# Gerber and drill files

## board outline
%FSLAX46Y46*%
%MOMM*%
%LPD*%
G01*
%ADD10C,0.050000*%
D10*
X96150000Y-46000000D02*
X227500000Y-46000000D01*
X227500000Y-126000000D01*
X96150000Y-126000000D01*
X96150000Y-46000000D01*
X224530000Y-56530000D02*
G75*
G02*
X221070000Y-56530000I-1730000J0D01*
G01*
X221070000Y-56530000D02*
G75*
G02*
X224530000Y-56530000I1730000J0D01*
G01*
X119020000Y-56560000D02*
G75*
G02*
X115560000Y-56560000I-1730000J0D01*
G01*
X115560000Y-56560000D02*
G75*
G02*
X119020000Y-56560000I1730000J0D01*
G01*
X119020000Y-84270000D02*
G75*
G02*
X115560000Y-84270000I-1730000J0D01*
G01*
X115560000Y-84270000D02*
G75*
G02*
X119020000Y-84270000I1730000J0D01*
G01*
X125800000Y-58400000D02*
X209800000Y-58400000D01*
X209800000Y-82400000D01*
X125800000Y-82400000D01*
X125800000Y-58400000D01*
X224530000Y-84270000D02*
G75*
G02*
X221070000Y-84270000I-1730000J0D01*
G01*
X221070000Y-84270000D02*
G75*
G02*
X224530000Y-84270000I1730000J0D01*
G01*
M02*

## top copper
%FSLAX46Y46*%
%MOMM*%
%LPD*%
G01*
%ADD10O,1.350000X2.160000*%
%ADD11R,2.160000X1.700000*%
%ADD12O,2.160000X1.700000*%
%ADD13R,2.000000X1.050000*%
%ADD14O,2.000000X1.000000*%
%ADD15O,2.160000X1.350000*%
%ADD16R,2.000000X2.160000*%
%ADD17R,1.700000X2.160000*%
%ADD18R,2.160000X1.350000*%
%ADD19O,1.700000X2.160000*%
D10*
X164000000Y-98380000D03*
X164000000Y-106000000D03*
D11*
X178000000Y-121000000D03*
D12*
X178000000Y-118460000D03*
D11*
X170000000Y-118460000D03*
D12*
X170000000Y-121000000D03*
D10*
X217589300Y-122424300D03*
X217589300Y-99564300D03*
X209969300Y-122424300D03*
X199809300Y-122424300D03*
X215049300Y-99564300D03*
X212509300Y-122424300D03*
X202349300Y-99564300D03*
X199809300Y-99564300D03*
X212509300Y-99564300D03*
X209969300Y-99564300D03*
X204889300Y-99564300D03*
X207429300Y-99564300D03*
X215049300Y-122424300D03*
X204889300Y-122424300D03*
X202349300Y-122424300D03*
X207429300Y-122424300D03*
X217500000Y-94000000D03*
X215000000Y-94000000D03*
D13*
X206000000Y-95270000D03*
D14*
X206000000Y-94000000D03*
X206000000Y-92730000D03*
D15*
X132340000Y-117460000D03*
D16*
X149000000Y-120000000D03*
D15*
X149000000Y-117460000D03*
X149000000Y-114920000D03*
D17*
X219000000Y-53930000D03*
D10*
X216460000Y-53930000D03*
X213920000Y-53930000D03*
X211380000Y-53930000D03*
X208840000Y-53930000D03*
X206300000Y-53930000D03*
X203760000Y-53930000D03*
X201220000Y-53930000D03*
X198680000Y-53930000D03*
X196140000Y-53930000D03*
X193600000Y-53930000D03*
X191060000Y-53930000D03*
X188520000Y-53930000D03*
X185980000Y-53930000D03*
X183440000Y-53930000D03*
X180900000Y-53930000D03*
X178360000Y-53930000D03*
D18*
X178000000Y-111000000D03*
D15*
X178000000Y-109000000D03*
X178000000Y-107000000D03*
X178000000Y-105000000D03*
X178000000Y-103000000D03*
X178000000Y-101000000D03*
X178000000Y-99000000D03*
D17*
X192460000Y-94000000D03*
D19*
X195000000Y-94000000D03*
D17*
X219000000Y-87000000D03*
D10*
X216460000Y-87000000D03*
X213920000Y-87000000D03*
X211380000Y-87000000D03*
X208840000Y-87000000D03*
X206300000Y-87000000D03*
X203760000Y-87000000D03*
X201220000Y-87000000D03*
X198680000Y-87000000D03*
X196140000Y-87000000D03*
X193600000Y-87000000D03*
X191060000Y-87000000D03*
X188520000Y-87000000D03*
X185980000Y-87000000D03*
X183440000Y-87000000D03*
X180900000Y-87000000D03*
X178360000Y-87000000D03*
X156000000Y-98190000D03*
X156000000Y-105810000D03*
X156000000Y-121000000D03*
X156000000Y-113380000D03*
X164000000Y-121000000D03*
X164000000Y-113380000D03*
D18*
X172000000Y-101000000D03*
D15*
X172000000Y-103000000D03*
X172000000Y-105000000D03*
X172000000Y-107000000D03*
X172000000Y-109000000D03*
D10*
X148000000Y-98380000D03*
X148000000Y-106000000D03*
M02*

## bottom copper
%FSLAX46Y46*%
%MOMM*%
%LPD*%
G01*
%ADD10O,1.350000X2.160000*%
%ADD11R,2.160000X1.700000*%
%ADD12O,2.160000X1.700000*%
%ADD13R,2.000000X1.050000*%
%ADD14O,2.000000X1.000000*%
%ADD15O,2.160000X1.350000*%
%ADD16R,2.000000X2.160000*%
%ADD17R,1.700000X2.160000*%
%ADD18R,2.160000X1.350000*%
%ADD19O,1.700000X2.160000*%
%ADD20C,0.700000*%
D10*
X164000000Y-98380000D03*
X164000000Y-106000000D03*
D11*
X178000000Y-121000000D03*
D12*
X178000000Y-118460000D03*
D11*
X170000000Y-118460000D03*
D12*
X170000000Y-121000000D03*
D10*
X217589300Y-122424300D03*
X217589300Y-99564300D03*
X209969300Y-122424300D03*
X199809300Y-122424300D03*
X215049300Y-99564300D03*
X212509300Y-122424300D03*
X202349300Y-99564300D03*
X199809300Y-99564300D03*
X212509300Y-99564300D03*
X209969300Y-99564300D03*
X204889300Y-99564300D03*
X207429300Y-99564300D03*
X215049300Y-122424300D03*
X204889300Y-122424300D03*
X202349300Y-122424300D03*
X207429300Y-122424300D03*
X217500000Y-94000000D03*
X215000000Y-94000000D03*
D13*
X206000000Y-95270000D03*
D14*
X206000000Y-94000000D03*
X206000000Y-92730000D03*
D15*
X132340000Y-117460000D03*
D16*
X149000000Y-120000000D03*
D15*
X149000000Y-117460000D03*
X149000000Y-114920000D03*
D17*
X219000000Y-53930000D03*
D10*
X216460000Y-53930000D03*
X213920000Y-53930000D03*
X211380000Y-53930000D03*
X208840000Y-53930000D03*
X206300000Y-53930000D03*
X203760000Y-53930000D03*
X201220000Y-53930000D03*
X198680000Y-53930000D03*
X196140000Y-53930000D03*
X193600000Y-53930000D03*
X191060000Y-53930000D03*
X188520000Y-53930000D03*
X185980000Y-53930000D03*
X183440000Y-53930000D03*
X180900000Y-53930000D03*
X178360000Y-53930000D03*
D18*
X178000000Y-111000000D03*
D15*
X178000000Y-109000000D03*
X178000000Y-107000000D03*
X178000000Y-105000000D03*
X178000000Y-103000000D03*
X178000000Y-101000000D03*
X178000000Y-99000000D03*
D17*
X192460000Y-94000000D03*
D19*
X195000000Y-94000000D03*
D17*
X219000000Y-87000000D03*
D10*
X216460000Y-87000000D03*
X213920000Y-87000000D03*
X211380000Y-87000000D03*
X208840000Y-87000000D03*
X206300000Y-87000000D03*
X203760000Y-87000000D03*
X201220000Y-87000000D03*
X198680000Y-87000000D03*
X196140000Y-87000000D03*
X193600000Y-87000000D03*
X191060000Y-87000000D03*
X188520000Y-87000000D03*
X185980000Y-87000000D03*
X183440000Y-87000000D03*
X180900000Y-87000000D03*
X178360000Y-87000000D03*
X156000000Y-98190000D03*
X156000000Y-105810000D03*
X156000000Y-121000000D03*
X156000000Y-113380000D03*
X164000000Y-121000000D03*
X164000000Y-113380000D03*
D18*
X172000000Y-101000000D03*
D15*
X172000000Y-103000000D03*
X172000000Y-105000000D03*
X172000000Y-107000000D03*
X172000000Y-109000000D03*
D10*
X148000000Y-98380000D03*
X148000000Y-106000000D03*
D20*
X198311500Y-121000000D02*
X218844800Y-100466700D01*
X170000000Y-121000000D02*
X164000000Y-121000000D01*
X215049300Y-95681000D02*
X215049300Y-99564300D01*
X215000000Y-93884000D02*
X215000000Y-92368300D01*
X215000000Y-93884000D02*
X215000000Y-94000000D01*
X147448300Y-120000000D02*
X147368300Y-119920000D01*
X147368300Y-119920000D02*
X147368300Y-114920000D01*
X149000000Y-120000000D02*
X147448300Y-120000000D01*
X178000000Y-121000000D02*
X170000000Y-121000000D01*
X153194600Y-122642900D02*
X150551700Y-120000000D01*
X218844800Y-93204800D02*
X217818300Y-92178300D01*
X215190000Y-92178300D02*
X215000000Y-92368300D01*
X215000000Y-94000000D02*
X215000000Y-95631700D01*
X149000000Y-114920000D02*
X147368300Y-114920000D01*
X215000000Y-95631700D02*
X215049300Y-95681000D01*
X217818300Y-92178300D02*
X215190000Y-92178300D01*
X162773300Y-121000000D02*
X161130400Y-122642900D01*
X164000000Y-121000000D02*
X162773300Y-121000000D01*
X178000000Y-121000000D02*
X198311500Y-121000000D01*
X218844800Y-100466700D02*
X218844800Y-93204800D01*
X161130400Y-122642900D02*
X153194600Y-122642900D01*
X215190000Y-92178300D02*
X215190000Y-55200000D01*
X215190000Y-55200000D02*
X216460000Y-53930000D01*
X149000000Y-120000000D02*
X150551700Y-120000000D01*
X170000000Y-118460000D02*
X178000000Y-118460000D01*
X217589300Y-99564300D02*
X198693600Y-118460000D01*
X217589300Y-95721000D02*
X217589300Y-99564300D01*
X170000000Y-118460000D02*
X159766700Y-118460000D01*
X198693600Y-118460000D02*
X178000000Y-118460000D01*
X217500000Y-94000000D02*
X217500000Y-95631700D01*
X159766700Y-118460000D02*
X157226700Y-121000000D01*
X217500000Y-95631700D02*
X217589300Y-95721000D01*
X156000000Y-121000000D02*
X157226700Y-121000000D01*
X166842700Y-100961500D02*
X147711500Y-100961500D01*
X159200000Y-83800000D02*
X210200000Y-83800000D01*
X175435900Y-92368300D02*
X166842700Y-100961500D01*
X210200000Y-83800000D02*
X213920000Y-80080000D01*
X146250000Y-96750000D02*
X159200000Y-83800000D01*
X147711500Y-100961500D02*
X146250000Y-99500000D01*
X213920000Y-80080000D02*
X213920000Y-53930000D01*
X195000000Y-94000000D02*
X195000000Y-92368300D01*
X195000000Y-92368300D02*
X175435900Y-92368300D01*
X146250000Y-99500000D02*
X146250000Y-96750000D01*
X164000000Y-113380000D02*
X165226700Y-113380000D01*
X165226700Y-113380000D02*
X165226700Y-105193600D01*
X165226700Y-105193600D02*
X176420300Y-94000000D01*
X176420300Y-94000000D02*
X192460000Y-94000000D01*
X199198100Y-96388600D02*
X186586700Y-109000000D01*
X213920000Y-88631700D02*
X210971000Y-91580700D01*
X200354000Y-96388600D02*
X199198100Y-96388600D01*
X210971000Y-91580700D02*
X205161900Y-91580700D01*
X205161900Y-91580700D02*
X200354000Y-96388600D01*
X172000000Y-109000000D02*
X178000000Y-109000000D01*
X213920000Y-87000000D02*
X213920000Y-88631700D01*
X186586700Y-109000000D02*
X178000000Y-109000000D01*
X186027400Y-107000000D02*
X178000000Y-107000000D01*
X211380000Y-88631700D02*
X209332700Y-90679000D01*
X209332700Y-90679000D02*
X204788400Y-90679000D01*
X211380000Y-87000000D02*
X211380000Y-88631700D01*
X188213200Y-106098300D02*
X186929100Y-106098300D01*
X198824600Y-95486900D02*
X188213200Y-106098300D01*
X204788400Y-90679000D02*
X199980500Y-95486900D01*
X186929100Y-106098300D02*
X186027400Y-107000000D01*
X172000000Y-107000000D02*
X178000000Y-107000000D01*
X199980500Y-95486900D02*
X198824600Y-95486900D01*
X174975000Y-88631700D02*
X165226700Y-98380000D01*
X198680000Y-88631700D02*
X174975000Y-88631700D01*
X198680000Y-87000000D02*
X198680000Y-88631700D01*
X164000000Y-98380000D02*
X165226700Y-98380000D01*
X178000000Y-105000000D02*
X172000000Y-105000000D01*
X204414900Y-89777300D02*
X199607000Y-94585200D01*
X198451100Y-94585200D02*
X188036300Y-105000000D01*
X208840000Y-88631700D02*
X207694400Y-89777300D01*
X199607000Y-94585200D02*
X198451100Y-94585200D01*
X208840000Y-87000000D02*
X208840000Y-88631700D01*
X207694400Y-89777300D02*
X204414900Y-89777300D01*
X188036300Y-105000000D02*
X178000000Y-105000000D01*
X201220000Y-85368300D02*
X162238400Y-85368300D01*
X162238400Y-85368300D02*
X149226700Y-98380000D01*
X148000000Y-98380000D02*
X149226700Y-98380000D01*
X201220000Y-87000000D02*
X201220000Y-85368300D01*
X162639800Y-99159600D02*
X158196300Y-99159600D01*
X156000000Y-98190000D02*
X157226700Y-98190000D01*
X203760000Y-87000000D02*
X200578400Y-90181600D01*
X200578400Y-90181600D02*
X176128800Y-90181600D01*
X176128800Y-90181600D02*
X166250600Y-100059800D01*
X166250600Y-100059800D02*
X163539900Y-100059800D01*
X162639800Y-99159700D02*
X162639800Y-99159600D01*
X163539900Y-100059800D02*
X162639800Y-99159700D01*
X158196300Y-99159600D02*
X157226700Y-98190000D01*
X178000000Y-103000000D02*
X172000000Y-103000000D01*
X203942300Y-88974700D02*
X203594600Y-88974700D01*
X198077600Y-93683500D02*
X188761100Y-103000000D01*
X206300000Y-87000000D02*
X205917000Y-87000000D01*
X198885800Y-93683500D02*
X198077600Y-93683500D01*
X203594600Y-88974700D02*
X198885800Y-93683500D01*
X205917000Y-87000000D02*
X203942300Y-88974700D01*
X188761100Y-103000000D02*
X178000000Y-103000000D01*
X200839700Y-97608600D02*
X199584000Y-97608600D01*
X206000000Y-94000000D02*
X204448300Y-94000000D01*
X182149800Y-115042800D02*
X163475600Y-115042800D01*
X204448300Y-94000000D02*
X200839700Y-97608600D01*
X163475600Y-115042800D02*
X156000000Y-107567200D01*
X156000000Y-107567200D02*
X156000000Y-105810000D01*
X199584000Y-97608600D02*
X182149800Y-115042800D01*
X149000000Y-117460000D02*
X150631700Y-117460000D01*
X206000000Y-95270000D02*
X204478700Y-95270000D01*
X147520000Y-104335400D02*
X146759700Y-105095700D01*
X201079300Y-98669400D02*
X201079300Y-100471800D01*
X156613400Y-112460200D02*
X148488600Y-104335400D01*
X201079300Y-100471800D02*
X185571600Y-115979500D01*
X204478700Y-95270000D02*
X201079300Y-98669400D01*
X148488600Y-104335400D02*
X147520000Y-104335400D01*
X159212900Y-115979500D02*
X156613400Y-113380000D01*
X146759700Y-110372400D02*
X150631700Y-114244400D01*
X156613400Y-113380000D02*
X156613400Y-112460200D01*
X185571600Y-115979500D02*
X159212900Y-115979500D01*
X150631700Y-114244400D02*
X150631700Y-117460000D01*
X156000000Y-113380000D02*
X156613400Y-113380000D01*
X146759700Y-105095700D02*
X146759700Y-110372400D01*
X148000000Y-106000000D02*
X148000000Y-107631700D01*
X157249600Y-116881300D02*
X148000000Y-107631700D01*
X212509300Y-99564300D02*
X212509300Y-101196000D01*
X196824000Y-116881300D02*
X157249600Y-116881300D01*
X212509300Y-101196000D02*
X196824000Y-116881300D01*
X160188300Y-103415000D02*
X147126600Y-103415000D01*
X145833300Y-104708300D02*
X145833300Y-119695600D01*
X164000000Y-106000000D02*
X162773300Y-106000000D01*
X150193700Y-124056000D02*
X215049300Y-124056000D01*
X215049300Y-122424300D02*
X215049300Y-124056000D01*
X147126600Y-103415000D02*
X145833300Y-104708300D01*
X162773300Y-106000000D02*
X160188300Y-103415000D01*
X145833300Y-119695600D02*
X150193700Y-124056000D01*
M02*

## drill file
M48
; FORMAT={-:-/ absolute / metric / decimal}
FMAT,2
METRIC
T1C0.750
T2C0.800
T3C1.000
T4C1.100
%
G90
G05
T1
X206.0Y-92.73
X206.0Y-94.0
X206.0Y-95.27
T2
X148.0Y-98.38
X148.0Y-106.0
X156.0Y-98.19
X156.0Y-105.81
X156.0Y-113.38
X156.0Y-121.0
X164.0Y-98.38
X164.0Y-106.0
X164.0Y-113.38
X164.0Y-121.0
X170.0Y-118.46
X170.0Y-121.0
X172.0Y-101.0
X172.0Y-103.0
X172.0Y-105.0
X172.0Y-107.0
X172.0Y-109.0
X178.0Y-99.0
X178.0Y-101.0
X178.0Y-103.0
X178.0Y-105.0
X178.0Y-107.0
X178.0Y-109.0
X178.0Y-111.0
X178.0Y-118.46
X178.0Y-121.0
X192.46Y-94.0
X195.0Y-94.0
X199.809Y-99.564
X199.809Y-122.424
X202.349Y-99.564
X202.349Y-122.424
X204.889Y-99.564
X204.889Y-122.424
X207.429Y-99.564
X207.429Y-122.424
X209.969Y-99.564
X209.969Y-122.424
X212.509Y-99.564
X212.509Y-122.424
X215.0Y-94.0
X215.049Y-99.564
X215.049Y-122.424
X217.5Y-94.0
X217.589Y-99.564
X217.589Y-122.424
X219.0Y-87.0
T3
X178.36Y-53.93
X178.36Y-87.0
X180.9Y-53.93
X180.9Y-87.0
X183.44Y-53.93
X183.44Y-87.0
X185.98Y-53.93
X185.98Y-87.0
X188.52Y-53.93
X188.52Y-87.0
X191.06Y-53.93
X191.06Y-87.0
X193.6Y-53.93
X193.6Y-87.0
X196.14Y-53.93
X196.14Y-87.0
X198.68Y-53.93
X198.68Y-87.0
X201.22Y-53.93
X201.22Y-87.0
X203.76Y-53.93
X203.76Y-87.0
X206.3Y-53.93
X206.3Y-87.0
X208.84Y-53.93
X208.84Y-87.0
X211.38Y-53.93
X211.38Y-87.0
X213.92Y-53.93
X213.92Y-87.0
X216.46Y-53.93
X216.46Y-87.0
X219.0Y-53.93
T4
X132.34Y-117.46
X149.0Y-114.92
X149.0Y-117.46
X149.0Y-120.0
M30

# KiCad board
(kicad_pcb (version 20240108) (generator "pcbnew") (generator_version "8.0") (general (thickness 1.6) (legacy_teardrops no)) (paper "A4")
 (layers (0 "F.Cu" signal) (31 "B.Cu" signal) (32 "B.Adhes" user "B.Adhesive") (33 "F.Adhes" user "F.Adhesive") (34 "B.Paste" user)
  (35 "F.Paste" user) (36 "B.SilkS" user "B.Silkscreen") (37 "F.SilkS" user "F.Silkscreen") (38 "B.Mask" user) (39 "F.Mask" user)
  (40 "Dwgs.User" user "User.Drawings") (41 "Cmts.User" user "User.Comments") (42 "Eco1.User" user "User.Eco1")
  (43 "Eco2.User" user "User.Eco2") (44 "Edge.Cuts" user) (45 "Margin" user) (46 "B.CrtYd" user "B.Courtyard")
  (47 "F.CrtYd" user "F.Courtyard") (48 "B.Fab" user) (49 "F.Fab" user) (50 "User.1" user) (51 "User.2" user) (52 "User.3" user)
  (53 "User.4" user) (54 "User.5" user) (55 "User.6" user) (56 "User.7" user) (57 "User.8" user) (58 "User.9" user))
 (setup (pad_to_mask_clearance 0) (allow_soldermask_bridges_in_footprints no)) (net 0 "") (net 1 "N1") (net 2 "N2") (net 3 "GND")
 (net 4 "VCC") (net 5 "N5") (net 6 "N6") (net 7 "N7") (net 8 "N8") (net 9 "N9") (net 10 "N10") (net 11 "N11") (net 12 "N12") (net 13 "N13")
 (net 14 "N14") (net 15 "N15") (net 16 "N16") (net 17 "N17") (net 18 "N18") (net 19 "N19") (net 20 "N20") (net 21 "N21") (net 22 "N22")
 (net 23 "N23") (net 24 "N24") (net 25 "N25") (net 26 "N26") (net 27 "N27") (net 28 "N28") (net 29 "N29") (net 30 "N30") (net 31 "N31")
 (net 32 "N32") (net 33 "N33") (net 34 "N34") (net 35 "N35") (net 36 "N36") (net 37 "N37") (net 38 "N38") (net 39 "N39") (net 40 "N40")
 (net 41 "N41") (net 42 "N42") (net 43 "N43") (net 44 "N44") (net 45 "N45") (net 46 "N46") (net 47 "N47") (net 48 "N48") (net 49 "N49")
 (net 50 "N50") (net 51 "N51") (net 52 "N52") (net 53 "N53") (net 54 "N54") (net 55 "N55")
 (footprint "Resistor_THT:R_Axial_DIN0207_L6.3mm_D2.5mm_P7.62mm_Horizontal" (layer "F.Cu") (at 164 98.38 -90)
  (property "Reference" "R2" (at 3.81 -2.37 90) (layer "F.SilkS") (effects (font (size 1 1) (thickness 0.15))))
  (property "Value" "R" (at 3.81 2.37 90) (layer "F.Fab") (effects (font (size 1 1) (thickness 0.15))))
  (pad "1" thru_hole oval (at 0 0 270) (size 2.16 1.35) (drill 0.8) (layers "*.Cu" "*.Mask") (remove_unused_layers no) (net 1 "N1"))
  (pad "2" thru_hole oval (at 7.62 0 270) (size 2.16 1.35) (drill 0.8) (layers "*.Cu" "*.Mask") (remove_unused_layers no) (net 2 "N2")))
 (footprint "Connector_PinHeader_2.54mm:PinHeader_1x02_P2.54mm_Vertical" (layer "F.Cu") (at 178 121 180)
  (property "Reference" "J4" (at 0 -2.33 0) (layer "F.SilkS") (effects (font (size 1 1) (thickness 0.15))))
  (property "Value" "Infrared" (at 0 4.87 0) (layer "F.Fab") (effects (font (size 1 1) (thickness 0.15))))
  (pad "1" thru_hole rect (at 0 0 180) (size 2.16 1.7) (drill 0.8) (layers "*.Cu" "*.Mask") (remove_unused_layers no) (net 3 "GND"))
  (pad "2" thru_hole oval (at 0 2.54 180) (size 2.16 1.7) (drill 0.8) (layers "*.Cu" "*.Mask") (remove_unused_layers no) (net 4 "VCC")))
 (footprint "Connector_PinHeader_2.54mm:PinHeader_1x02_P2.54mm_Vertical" (layer "F.Cu") (at 170 118.46)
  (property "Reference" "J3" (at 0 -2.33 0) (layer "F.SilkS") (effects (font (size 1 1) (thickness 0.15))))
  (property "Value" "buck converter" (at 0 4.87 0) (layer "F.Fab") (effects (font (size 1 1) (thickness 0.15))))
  (pad "1" thru_hole rect (at 0 0) (size 2.16 1.7) (drill 0.8) (layers "*.Cu" "*.Mask") (remove_unused_layers no) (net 4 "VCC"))
  (pad "2" thru_hole oval (at 0 2.54) (size 2.16 1.7) (drill 0.8) (layers "*.Cu" "*.Mask") (remove_unused_layers no) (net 3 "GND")))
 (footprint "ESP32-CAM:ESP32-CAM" (layer "F.Cu") (at 193.4593 110.9943 90)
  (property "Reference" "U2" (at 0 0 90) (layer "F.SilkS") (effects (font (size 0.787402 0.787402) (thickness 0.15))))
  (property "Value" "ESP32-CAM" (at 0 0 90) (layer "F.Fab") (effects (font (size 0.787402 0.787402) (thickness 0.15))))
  (pad "3V3" thru_hole oval (at -11.43 24.13 90) (size 2.16 1.35) (drill 0.8) (layers "*.Cu" "*.Mask") (remove_unused_layers no)
   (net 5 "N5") (solder_mask_margin 0.102))
  (pad "5V" thru_hole oval (at 11.43 24.13 90) (size 2.16 1.35) (drill 0.8) (layers "*.Cu" "*.Mask") (remove_unused_layers no) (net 4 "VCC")
   (solder_mask_margin 0.102))
  (pad "GND" thru_hole oval (at -11.43 16.51 90) (size 2.16 1.35) (drill 0.8) (layers "*.Cu" "*.Mask") (remove_unused_layers no)
   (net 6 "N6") (solder_mask_margin 0.102))
  (pad "GND1" thru_hole oval (at -11.43 6.35 90) (size 2.16 1.35) (drill 0.8) (layers "*.Cu" "*.Mask") (remove_unused_layers no)
   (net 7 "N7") (solder_mask_margin 0.102))
  (pad "GND2" thru_hole oval (at 11.43 21.59 90) (size 2.16 1.35) (drill 0.8) (layers "*.Cu" "*.Mask") (remove_unused_layers no)
   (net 3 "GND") (solder_mask_margin 0.102))
  (pad "IO0" thru_hole oval (at -11.43 19.05 90) (size 2.16 1.35) (drill 0.8) (layers "*.Cu" "*.Mask") (remove_unused_layers no)
   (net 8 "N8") (solder_mask_margin 0.102))
  (pad "IO2" thru_hole oval (at 11.43 8.89 90) (size 2.16 1.35) (drill 0.8) (layers "*.Cu" "*.Mask") (remove_unused_layers no) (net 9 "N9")
   (solder_mask_margin 0.102))
  (pad "IO4" thru_hole oval (at 11.43 6.35 90) (size 2.16 1.35) (drill 0.8) (layers "*.Cu" "*.Mask") (remove_unused_layers no)
   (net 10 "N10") (solder_mask_margin 0.102))
  (pad "IO12" thru_hole oval (at 11.43 19.05 90) (size 2.16 1.35) (drill 0.8) (layers "*.Cu" "*.Mask") (remove_unused_layers no)
   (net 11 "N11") (solder_mask_margin 0.102))
  (pad "IO13" thru_hole oval (at 11.43 16.51 90) (size 2.16 1.35) (drill 0.8) (layers "*.Cu" "*.Mask") (remove_unused_layers no)
   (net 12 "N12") (solder_mask_margin 0.102))
  (pad "IO14" thru_hole oval (at 11.43 11.43 90) (size 2.16 1.35) (drill 0.8) (layers "*.Cu" "*.Mask") (remove_unused_layers no)
   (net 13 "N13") (solder_mask_margin 0.102))
  (pad "IO15" thru_hole oval (at 11.43 13.97 90) (size 2.16 1.35) (drill 0.8) (layers "*.Cu" "*.Mask") (remove_unused_layers no)
   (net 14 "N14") (solder_mask_margin 0.102))
  (pad "IO16" thru_hole oval (at -11.43 21.59 90) (size 2.16 1.35) (drill 0.8) (layers "*.Cu" "*.Mask") (remove_unused_layers no)
   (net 2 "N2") (solder_mask_margin 0.102))
  (pad "U0R" thru_hole oval (at -11.43 11.43 90) (size 2.16 1.35) (drill 0.8) (layers "*.Cu" "*.Mask") (remove_unused_layers no)
   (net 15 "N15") (solder_mask_margin 0.102))
  (pad "U0T" thru_hole oval (at -11.43 8.89 90) (size 2.16 1.35) (drill 0.8) (layers "*.Cu" "*.Mask") (remove_unused_layers no)
   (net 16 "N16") (solder_mask_margin 0.102))
  (pad "VOUT" thru_hole oval (at -11.43 13.97 90) (size 2.16 1.35) (drill 0.8) (layers "*.Cu" "*.Mask") (remove_unused_layers no)
   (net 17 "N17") (solder_mask_margin 0.102)))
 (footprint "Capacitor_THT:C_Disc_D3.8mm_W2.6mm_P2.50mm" (layer "F.Cu") (at 217.5 94 180)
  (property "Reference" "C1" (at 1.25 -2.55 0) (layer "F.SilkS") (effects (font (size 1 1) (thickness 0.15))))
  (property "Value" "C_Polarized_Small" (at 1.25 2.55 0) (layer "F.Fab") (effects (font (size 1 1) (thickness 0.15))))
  (pad "1" thru_hole oval (at 0 0 180) (size 1.35 2.16) (drill 0.8) (layers "*.Cu" "*.Mask") (remove_unused_layers no) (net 4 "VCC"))
  (pad "2" thru_hole oval (at 2.5 0 180) (size 1.35 2.16) (drill 0.8) (layers "*.Cu" "*.Mask") (remove_unused_layers no) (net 3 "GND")))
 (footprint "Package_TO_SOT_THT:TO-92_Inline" (layer "F.Cu") (at 206 95.27 90)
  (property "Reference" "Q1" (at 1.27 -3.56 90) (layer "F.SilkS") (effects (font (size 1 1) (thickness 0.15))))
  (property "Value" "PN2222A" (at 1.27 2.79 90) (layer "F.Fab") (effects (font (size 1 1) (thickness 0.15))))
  (pad "1" thru_hole rect (at 0 0 90) (size 1.05 2) (drill 0.75) (layers "*.Cu" "*.Mask") (remove_unused_layers no) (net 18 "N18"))
  (pad "2" thru_hole oval (at 1.27 0 90) (size 1 2) (drill 0.75) (layers "*.Cu" "*.Mask") (remove_unused_layers no) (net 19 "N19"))
  (pad "3" thru_hole oval (at 2.54 0 90) (size 1 2) (drill 0.75) (layers "*.Cu" "*.Mask") (remove_unused_layers no) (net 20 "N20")))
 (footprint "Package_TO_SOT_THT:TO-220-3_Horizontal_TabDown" (layer "F.Cu") (at 149 120 90)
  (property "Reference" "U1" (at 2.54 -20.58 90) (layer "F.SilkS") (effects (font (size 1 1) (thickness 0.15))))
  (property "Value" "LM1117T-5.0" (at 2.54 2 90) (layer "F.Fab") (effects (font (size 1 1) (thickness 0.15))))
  (pad "" thru_hole oval (at 2.54 -16.66 90) (size 1.35 2.16) (drill 1.1) (layers "*.Cu" "*.Mask") (remove_unused_layers no))
  (pad "1" thru_hole rect (at 0 0 90) (size 2.16 2) (drill 1.1) (layers "*.Cu" "*.Mask") (remove_unused_layers no) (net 3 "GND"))
  (pad "2" thru_hole oval (at 2.54 0 90) (size 1.35 2.16) (drill 1.1) (layers "*.Cu" "*.Mask") (remove_unused_layers no) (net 18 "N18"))
  (pad "3" thru_hole oval (at 5.08 0 90) (size 1.35 2.16) (drill 1.1) (layers "*.Cu" "*.Mask") (remove_unused_layers no) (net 3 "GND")))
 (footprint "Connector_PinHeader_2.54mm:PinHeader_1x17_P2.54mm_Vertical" (layer "F.Cu") (at 219 53.93 -90)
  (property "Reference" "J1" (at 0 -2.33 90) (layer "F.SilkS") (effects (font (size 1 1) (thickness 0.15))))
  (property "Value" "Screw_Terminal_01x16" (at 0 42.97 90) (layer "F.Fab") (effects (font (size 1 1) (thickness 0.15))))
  (pad "1" thru_hole rect (at 0 0 270) (size 2.16 1.7) (drill 1) (layers "*.Cu" "*.Mask") (remove_unused_layers no) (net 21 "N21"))
  (pad "2" thru_hole oval (at 0 2.54 270) (size 2.16 1.35) (drill 1) (layers "*.Cu" "*.Mask") (remove_unused_layers no) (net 3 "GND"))
  (pad "3" thru_hole oval (at 0 5.08 270) (size 2.16 1.35) (drill 1) (layers "*.Cu" "*.Mask") (remove_unused_layers no) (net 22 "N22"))
  (pad "4" thru_hole oval (at 0 7.62 270) (size 2.16 1.35) (drill 1) (layers "*.Cu" "*.Mask") (remove_unused_layers no) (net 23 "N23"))
  (pad "5" thru_hole oval (at 0 10.16 270) (size 2.16 1.35) (drill 1) (layers "*.Cu" "*.Mask") (remove_unused_layers no) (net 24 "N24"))
  (pad "6" thru_hole oval (at 0 12.7 270) (size 2.16 1.35) (drill 1) (layers "*.Cu" "*.Mask") (remove_unused_layers no) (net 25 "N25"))
  (pad "7" thru_hole oval (at 0 15.24 270) (size 2.16 1.35) (drill 1) (layers "*.Cu" "*.Mask") (remove_unused_layers no) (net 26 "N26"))
  (pad "8" thru_hole oval (at 0 17.78 270) (size 2.16 1.35) (drill 1) (layers "*.Cu" "*.Mask") (remove_unused_layers no) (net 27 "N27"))
  (pad "9" thru_hole oval (at 0 20.32 270) (size 2.16 1.35) (drill 1) (layers "*.Cu" "*.Mask") (remove_unused_layers no) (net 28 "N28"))
  (pad "10" thru_hole oval (at 0 22.86 270) (size 2.16 1.35) (drill 1) (layers "*.Cu" "*.Mask") (remove_unused_layers no) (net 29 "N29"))
  (pad "11" thru_hole oval (at 0 25.4 270) (size 2.16 1.35) (drill 1) (layers "*.Cu" "*.Mask") (remove_unused_layers no) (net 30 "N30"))
  (pad "12" thru_hole oval (at 0 27.94 270) (size 2.16 1.35) (drill 1) (layers "*.Cu" "*.Mask") (remove_unused_layers no) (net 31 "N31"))
  (pad "13" thru_hole oval (at 0 30.48 270) (size 2.16 1.35) (drill 1) (layers "*.Cu" "*.Mask") (remove_unused_layers no) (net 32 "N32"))
  (pad "14" thru_hole oval (at 0 33.02 270) (size 2.16 1.35) (drill 1) (layers "*.Cu" "*.Mask") (remove_unused_layers no) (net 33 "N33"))
  (pad "15" thru_hole oval (at 0 35.56 270) (size 2.16 1.35) (drill 1) (layers "*.Cu" "*.Mask") (remove_unused_layers no) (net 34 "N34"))
  (pad "16" thru_hole oval (at 0 38.1 270) (size 2.16 1.35) (drill 1) (layers "*.Cu" "*.Mask") (remove_unused_layers no) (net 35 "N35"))
  (pad "17" thru_hole oval (at 0 40.64 270) (size 2.16 1.35) (drill 1) (layers "*.Cu" "*.Mask") (remove_unused_layers no)))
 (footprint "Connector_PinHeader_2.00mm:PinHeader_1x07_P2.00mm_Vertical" (layer "F.Cu") (at 178 111 180)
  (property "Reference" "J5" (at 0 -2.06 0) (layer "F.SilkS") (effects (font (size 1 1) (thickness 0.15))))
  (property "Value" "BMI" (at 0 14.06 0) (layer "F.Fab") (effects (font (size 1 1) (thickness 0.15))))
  (pad "1" thru_hole rect (at 0 0 180) (size 2.16 1.35) (drill 0.8) (layers "*.Cu" "*.Mask") (remove_unused_layers no) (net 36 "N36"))
  (pad "2" thru_hole oval (at 0 2 180) (size 2.16 1.35) (drill 0.8) (layers "*.Cu" "*.Mask") (remove_unused_layers no) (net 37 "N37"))
  (pad "3" thru_hole oval (at 0 4 180) (size 2.16 1.35) (drill 0.8) (layers "*.Cu" "*.Mask") (remove_unused_layers no) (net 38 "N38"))
  (pad "4" thru_hole oval (at 0 6 180) (size 2.16 1.35) (drill 0.8) (layers "*.Cu" "*.Mask") (remove_unused_layers no) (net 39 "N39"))
  (pad "5" thru_hole oval (at 0 8 180) (size 2.16 1.35) (drill 0.8) (layers "*.Cu" "*.Mask") (remove_unused_layers no) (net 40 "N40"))
  (pad "6" thru_hole oval (at 0 10 180) (size 2.16 1.35) (drill 0.8) (layers "*.Cu" "*.Mask") (remove_unused_layers no) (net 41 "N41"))
  (pad "7" thru_hole oval (at 0 12 180) (size 2.16 1.35) (drill 0.8) (layers "*.Cu" "*.Mask") (remove_unused_layers no) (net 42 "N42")))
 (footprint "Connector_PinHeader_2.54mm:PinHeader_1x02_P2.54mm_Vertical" (layer "F.Cu") (at 192.46 94 90)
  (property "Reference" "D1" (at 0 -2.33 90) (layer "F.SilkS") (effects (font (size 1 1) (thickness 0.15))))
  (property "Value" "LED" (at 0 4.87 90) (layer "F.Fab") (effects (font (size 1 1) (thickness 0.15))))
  (pad "1" thru_hole rect (at 0 0 90) (size 2.16 1.7) (drill 0.8) (layers "*.Cu" "*.Mask") (remove_unused_layers no) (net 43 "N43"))
  (pad "2" thru_hole oval (at 0 2.54 90) (size 2.16 1.7) (drill 0.8) (layers "*.Cu" "*.Mask") (remove_unused_layers no) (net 22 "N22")))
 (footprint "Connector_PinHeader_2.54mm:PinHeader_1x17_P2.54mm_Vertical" (layer "F.Cu") (at 219 87 -90)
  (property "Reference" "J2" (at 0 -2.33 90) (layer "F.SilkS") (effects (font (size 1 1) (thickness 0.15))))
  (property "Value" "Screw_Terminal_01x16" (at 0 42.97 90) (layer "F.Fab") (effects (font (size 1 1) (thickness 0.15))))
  (pad "1" thru_hole rect (at 0 0 270) (size 2.16 1.7) (drill 0.8) (layers "*.Cu" "*.Mask") (remove_unused_layers no) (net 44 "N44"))
  (pad "2" thru_hole oval (at 0 2.54 270) (size 2.16 1.35) (drill 1) (layers "*.Cu" "*.Mask") (remove_unused_layers no) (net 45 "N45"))
  (pad "3" thru_hole oval (at 0 5.08 270) (size 2.16 1.35) (drill 1) (layers "*.Cu" "*.Mask") (remove_unused_layers no) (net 37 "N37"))
  (pad "4" thru_hole oval (at 0 7.62 270) (size 2.16 1.35) (drill 1) (layers "*.Cu" "*.Mask") (remove_unused_layers no) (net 38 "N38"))
  (pad "5" thru_hole oval (at 0 10.16 270) (size 2.16 1.35) (drill 1) (layers "*.Cu" "*.Mask") (remove_unused_layers no) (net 39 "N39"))
  (pad "6" thru_hole oval (at 0 12.7 270) (size 2.16 1.35) (drill 1) (layers "*.Cu" "*.Mask") (remove_unused_layers no) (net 40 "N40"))
  (pad "7" thru_hole oval (at 0 15.24 270) (size 2.16 1.35) (drill 1) (layers "*.Cu" "*.Mask") (remove_unused_layers no) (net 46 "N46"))
  (pad "8" thru_hole oval (at 0 17.78 270) (size 2.16 1.35) (drill 1) (layers "*.Cu" "*.Mask") (remove_unused_layers no) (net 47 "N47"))
  (pad "9" thru_hole oval (at 0 20.32 270) (size 2.16 1.35) (drill 1) (layers "*.Cu" "*.Mask") (remove_unused_layers no) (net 1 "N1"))
  (pad "10" thru_hole oval (at 0 22.86 270) (size 2.16 1.35) (drill 1) (layers "*.Cu" "*.Mask") (remove_unused_layers no) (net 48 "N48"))
  (pad "11" thru_hole oval (at 0 25.4 270) (size 2.16 1.35) (drill 1) (layers "*.Cu" "*.Mask") (remove_unused_layers no) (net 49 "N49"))
  (pad "12" thru_hole oval (at 0 27.94 270) (size 2.16 1.35) (drill 1) (layers "*.Cu" "*.Mask") (remove_unused_layers no) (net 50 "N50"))
  (pad "13" thru_hole oval (at 0 30.48 270) (size 2.16 1.35) (drill 1) (layers "*.Cu" "*.Mask") (remove_unused_layers no) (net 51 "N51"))
  (pad "14" thru_hole oval (at 0 33.02 270) (size 2.16 1.35) (drill 1) (layers "*.Cu" "*.Mask") (remove_unused_layers no) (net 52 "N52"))
  (pad "15" thru_hole oval (at 0 35.56 270) (size 2.16 1.35) (drill 1) (layers "*.Cu" "*.Mask") (remove_unused_layers no) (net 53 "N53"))
  (pad "16" thru_hole oval (at 0 38.1 270) (size 2.16 1.35) (drill 1) (layers "*.Cu" "*.Mask") (remove_unused_layers no) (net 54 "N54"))
  (pad "17" thru_hole oval (at 0 40.64 270) (size 2.16 1.35) (drill 1) (layers "*.Cu" "*.Mask") (remove_unused_layers no)))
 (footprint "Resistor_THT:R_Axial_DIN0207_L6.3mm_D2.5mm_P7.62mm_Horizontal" (layer "F.Cu") (at 156 98.19 -90)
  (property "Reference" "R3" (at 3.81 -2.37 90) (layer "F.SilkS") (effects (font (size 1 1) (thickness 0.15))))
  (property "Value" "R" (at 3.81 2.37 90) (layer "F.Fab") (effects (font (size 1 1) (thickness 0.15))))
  (pad "1" thru_hole oval (at 0 0 270) (size 2.16 1.35) (drill 0.8) (layers "*.Cu" "*.Mask") (remove_unused_layers no) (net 46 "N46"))
  (pad "2" thru_hole oval (at 7.62 0 270) (size 2.16 1.35) (drill 0.8) (layers "*.Cu" "*.Mask") (remove_unused_layers no) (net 19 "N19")))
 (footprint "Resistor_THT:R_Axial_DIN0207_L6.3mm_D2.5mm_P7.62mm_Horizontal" (layer "F.Cu") (at 156 121 90)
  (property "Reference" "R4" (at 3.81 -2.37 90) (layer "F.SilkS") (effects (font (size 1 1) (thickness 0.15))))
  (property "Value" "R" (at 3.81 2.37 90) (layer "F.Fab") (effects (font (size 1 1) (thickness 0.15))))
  (pad "1" thru_hole oval (at 0 0 90) (size 2.16 1.35) (drill 0.8) (layers "*.Cu" "*.Mask") (remove_unused_layers no) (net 4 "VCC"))
  (pad "2" thru_hole oval (at 7.62 0 90) (size 2.16 1.35) (drill 0.8) (layers "*.Cu" "*.Mask") (remove_unused_layers no) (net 18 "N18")))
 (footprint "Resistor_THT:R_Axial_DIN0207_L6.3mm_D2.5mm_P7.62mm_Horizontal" (layer "F.Cu") (at 164 121 90)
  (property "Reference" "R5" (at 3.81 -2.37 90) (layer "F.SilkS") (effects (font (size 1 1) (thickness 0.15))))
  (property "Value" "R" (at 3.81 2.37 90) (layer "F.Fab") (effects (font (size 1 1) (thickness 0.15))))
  (pad "1" thru_hole oval (at 0 0 90) (size 2.16 1.35) (drill 0.8) (layers "*.Cu" "*.Mask") (remove_unused_layers no) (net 3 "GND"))
  (pad "2" thru_hole oval (at 7.62 0 90) (size 2.16 1.35) (drill 0.8) (layers "*.Cu" "*.Mask") (remove_unused_layers no) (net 43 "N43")))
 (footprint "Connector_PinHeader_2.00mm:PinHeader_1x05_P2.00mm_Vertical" (layer "F.Cu") (at 172 101)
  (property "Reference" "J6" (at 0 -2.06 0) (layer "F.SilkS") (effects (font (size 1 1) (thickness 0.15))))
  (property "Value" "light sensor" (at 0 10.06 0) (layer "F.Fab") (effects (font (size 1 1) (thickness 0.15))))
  (pad "1" thru_hole rect (at 0 0) (size 2.16 1.35) (drill 0.8) (layers "*.Cu" "*.Mask") (remove_unused_layers no) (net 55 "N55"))
  (pad "2" thru_hole oval (at 0 2) (size 2.16 1.35) (drill 0.8) (layers "*.Cu" "*.Mask") (remove_unused_layers no) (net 40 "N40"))
  (pad "3" thru_hole oval (at 0 4) (size 2.16 1.35) (drill 0.8) (layers "*.Cu" "*.Mask") (remove_unused_layers no) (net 39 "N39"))
  (pad "4" thru_hole oval (at 0 6) (size 2.16 1.35) (drill 0.8) (layers "*.Cu" "*.Mask") (remove_unused_layers no) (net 38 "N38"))
  (pad "5" thru_hole oval (at 0 8) (size 2.16 1.35) (drill 0.8) (layers "*.Cu" "*.Mask") (remove_unused_layers no) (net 37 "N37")))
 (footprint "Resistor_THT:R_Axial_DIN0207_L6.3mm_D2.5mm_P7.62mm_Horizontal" (layer "F.Cu") (at 148 98.38 -90)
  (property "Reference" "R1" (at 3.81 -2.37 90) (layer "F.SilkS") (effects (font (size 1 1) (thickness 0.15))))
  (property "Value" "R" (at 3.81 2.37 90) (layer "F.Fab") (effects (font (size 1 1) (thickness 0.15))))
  (pad "1" thru_hole oval (at 0 0 270) (size 2.16 1.35) (drill 0.8) (layers "*.Cu" "*.Mask") (remove_unused_layers no) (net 47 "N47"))
  (pad "2" thru_hole oval (at 7.62 0 270) (size 2.16 1.35) (drill 0.8) (layers "*.Cu" "*.Mask") (remove_unused_layers no) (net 11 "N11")))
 (gr_rect (start 96.15 46) (end 227.5 126) (stroke (width 0.05) (type default)) (fill none) (layer "Edge.Cuts"))
 (gr_circle (center 222.8 56.53) (end 221.07 56.53) (stroke (width 0.05) (type default)) (fill none) (layer "Edge.Cuts"))
 (gr_circle (center 117.29 56.56) (end 115.56 56.56) (stroke (width 0.05) (type default)) (fill none) (layer "Edge.Cuts"))
 (gr_circle (center 117.29 84.27) (end 115.56 84.27) (stroke (width 0.05) (type default)) (fill none) (layer "Edge.Cuts"))
 (gr_rect (start 125.8 58.4) (end 209.8 82.4) (stroke (width 0.05) (type default)) (fill none) (layer "Edge.Cuts"))
 (gr_circle (center 222.8 84.27) (end 221.07 84.27) (stroke (width 0.05) (type default)) (fill none) (layer "Edge.Cuts"))
 (segment (start 198.3115 121) (end 218.8448 100.4667) (width 0.7) (layer "B.Cu") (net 3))
 (segment (start 170 121) (end 164 121) (width 0.7) (layer "B.Cu") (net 3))
 (segment (start 215.0493 95.681) (end 215.0493 99.5643) (width 0.7) (layer "B.Cu") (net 3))
 (segment (start 215 93.884) (end 215 92.3683) (width 0.7) (layer "B.Cu") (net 3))
 (segment (start 215 93.884) (end 215 94) (width 0.7) (layer "B.Cu") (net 3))
 (segment (start 147.4483 120) (end 147.3683 119.92) (width 0.7) (layer "B.Cu") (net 3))
 (segment (start 147.3683 119.92) (end 147.3683 114.92) (width 0.7) (layer "B.Cu") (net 3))
 (segment (start 149 120) (end 147.4483 120) (width 0.7) (layer "B.Cu") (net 3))
 (segment (start 178 121) (end 170 121) (width 0.7) (layer "B.Cu") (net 3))
 (segment (start 153.1946 122.6429) (end 150.5517 120) (width 0.7) (layer "B.Cu") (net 3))
 (segment (start 218.8448 93.2048) (end 217.8183 92.1783) (width 0.7) (layer "B.Cu") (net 3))
 (segment (start 215.19 92.1783) (end 215 92.3683) (width 0.7) (layer "B.Cu") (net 3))
 (segment (start 215 94) (end 215 95.6317) (width 0.7) (layer "B.Cu") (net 3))
 (segment (start 149 114.92) (end 147.3683 114.92) (width 0.7) (layer "B.Cu") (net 3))
 (segment (start 215 95.6317) (end 215.0493 95.681) (width 0.7) (layer "B.Cu") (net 3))
 (segment (start 217.8183 92.1783) (end 215.19 92.1783) (width 0.7) (layer "B.Cu") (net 3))
 (segment (start 162.7733 121) (end 161.1304 122.6429) (width 0.7) (layer "B.Cu") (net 3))
 (segment (start 164 121) (end 162.7733 121) (width 0.7) (layer "B.Cu") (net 3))
 (segment (start 178 121) (end 198.3115 121) (width 0.7) (layer "B.Cu") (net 3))
 (segment (start 218.8448 100.4667) (end 218.8448 93.2048) (width 0.7) (layer "B.Cu") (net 3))
 (segment (start 161.1304 122.6429) (end 153.1946 122.6429) (width 0.7) (layer "B.Cu") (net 3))
 (segment (start 215.19 92.1783) (end 215.19 55.2) (width 0.7) (layer "B.Cu") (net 3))
 (segment (start 215.19 55.2) (end 216.46 53.93) (width 0.7) (layer "B.Cu") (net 3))
 (segment (start 149 120) (end 150.5517 120) (width 0.7) (layer "B.Cu") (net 3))
 (segment (start 170 118.46) (end 178 118.46) (width 0.7) (layer "B.Cu") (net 4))
 (segment (start 217.5893 99.5643) (end 198.6936 118.46) (width 0.7) (layer "B.Cu") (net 4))
 (segment (start 217.5893 95.721) (end 217.5893 99.5643) (width 0.7) (layer "B.Cu") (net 4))
 (segment (start 170 118.46) (end 159.7667 118.46) (width 0.7) (layer "B.Cu") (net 4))
 (segment (start 198.6936 118.46) (end 178 118.46) (width 0.7) (layer "B.Cu") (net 4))
 (segment (start 217.5 94) (end 217.5 95.6317) (width 0.7) (layer "B.Cu") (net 4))
 (segment (start 159.7667 118.46) (end 157.2267 121) (width 0.7) (layer "B.Cu") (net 4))
 (segment (start 217.5 95.6317) (end 217.5893 95.721) (width 0.7) (layer "B.Cu") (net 4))
 (segment (start 156 121) (end 157.2267 121) (width 0.7) (layer "B.Cu") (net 4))
 (segment (start 166.8427 100.9615) (end 147.7115 100.9615) (width 0.7) (layer "B.Cu") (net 22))
 (segment (start 159.2 83.8) (end 210.2 83.8) (width 0.7) (layer "B.Cu") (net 22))
 (segment (start 175.4359 92.3683) (end 166.8427 100.9615) (width 0.7) (layer "B.Cu") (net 22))
 (segment (start 210.2 83.8) (end 213.92 80.08) (width 0.7) (layer "B.Cu") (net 22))
 (segment (start 146.25 96.75) (end 159.2 83.8) (width 0.7) (layer "B.Cu") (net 22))
 (segment (start 147.7115 100.9615) (end 146.25 99.5) (width 0.7) (layer "B.Cu") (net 22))
 (segment (start 213.92 80.08) (end 213.92 53.93) (width 0.7) (layer "B.Cu") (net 22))
 (segment (start 195 94) (end 195 92.3683) (width 0.7) (layer "B.Cu") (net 22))
 (segment (start 195 92.3683) (end 175.4359 92.3683) (width 0.7) (layer "B.Cu") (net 22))
 (segment (start 146.25 99.5) (end 146.25 96.75) (width 0.7) (layer "B.Cu") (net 22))
 (segment (start 164 113.38) (end 165.2267 113.38) (width 0.7) (layer "B.Cu") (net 43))
 (segment (start 165.2267 113.38) (end 165.2267 105.1936) (width 0.7) (layer "B.Cu") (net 43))
 (segment (start 165.2267 105.1936) (end 176.4203 94) (width 0.7) (layer "B.Cu") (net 43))
 (segment (start 176.4203 94) (end 192.46 94) (width 0.7) (layer "B.Cu") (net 43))
 (segment (start 199.1981 96.3886) (end 186.5867 109) (width 0.7) (layer "B.Cu") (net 37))
 (segment (start 213.92 88.6317) (end 210.971 91.5807) (width 0.7) (layer "B.Cu") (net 37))
 (segment (start 200.354 96.3886) (end 199.1981 96.3886) (width 0.7) (layer "B.Cu") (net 37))
 (segment (start 210.971 91.5807) (end 205.1619 91.5807) (width 0.7) (layer "B.Cu") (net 37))
 (segment (start 205.1619 91.5807) (end 200.354 96.3886) (width 0.7) (layer "B.Cu") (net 37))
 (segment (start 172 109) (end 178 109) (width 0.7) (layer "B.Cu") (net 37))
 (segment (start 213.92 87) (end 213.92 88.6317) (width 0.7) (layer "B.Cu") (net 37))
 (segment (start 186.5867 109) (end 178 109) (width 0.7) (layer "B.Cu") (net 37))
 (segment (start 186.0274 107) (end 178 107) (width 0.7) (layer "B.Cu") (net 38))
 (segment (start 211.38 88.6317) (end 209.3327 90.679) (width 0.7) (layer "B.Cu") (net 38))
 (segment (start 209.3327 90.679) (end 204.7884 90.679) (width 0.7) (layer "B.Cu") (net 38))
 (segment (start 211.38 87) (end 211.38 88.6317) (width 0.7) (layer "B.Cu") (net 38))
 (segment (start 188.2132 106.0983) (end 186.9291 106.0983) (width 0.7) (layer "B.Cu") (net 38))
 (segment (start 198.8246 95.4869) (end 188.2132 106.0983) (width 0.7) (layer "B.Cu") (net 38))
 (segment (start 204.7884 90.679) (end 199.9805 95.4869) (width 0.7) (layer "B.Cu") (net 38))
 (segment (start 186.9291 106.0983) (end 186.0274 107) (width 0.7) (layer "B.Cu") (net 38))
 (segment (start 172 107) (end 178 107) (width 0.7) (layer "B.Cu") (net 38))
 (segment (start 199.9805 95.4869) (end 198.8246 95.4869) (width 0.7) (layer "B.Cu") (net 38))
 (segment (start 174.975 88.6317) (end 165.2267 98.38) (width 0.7) (layer "B.Cu") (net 1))
 (segment (start 198.68 88.6317) (end 174.975 88.6317) (width 0.7) (layer "B.Cu") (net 1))
 (segment (start 198.68 87) (end 198.68 88.6317) (width 0.7) (layer "B.Cu") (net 1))
 (segment (start 164 98.38) (end 165.2267 98.38) (width 0.7) (layer "B.Cu") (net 1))
 (segment (start 178 105) (end 172 105) (width 0.7) (layer "B.Cu") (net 39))
 (segment (start 204.4149 89.7773) (end 199.607 94.5852) (width 0.7) (layer "B.Cu") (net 39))
 (segment (start 198.4511 94.5852) (end 188.0363 105) (width 0.7) (layer "B.Cu") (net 39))
 (segment (start 208.84 88.6317) (end 207.6944 89.7773) (width 0.7) (layer "B.Cu") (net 39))
 (segment (start 199.607 94.5852) (end 198.4511 94.5852) (width 0.7) (layer "B.Cu") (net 39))
 (segment (start 208.84 87) (end 208.84 88.6317) (width 0.7) (layer "B.Cu") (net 39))
 (segment (start 207.6944 89.7773) (end 204.4149 89.7773) (width 0.7) (layer "B.Cu") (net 39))
 (segment (start 188.0363 105) (end 178 105) (width 0.7) (layer "B.Cu") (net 39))
 (segment (start 201.22 85.3683) (end 162.2384 85.3683) (width 0.7) (layer "B.Cu") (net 47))
 (segment (start 162.2384 85.3683) (end 149.2267 98.38) (width 0.7) (layer "B.Cu") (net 47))
 (segment (start 148 98.38) (end 149.2267 98.38) (width 0.7) (layer "B.Cu") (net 47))
 (segment (start 201.22 87) (end 201.22 85.3683) (width 0.7) (layer "B.Cu") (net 47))
 (segment (start 162.6398 99.1596) (end 158.1963 99.1596) (width 0.7) (layer "B.Cu") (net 46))
 (segment (start 156 98.19) (end 157.2267 98.19) (width 0.7) (layer "B.Cu") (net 46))
 (segment (start 203.76 87) (end 200.5784 90.1816) (width 0.7) (layer "B.Cu") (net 46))
 (segment (start 200.5784 90.1816) (end 176.1288 90.1816) (width 0.7) (layer "B.Cu") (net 46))
 (segment (start 176.1288 90.1816) (end 166.2506 100.0598) (width 0.7) (layer "B.Cu") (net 46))
 (segment (start 166.2506 100.0598) (end 163.5399 100.0598) (width 0.7) (layer "B.Cu") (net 46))
 (segment (start 162.6398 99.1597) (end 162.6398 99.1596) (width 0.7) (layer "B.Cu") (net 46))
 (segment (start 163.5399 100.0598) (end 162.6398 99.1597) (width 0.7) (layer "B.Cu") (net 46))
 (segment (start 158.1963 99.1596) (end 157.2267 98.19) (width 0.7) (layer "B.Cu") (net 46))
 (segment (start 178 103) (end 172 103) (width 0.7) (layer "B.Cu") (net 40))
 (segment (start 203.9423 88.9747) (end 203.5946 88.9747) (width 0.7) (layer "B.Cu") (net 40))
 (segment (start 198.0776 93.6835) (end 188.7611 103) (width 0.7) (layer "B.Cu") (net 40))
 (segment (start 206.3 87) (end 205.917 87) (width 0.7) (layer "B.Cu") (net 40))
 (segment (start 198.8858 93.6835) (end 198.0776 93.6835) (width 0.7) (layer "B.Cu") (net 40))
 (segment (start 203.5946 88.9747) (end 198.8858 93.6835) (width 0.7) (layer "B.Cu") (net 40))
 (segment (start 205.917 87) (end 203.9423 88.9747) (width 0.7) (layer "B.Cu") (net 40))
 (segment (start 188.7611 103) (end 178 103) (width 0.7) (layer "B.Cu") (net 40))
 (segment (start 200.8397 97.6086) (end 199.584 97.6086) (width 0.7) (layer "B.Cu") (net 19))
 (segment (start 206 94) (end 204.4483 94) (width 0.7) (layer "B.Cu") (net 19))
 (segment (start 182.1498 115.0428) (end 163.4756 115.0428) (width 0.7) (layer "B.Cu") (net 19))
 (segment (start 204.4483 94) (end 200.8397 97.6086) (width 0.7) (layer "B.Cu") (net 19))
 (segment (start 163.4756 115.0428) (end 156 107.5672) (width 0.7) (layer "B.Cu") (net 19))
 (segment (start 156 107.5672) (end 156 105.81) (width 0.7) (layer "B.Cu") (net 19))
 (segment (start 199.584 97.6086) (end 182.1498 115.0428) (width 0.7) (layer "B.Cu") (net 19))
 (segment (start 149 117.46) (end 150.6317 117.46) (width 0.7) (layer "B.Cu") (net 18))
 (segment (start 206 95.27) (end 204.4787 95.27) (width 0.7) (layer "B.Cu") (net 18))
 (segment (start 147.52 104.3354) (end 146.7597 105.0957) (width 0.7) (layer "B.Cu") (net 18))
 (segment (start 201.0793 98.6694) (end 201.0793 100.4718) (width 0.7) (layer "B.Cu") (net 18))
 (segment (start 156.6134 112.4602) (end 148.4886 104.3354) (width 0.7) (layer "B.Cu") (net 18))
 (segment (start 201.0793 100.4718) (end 185.5716 115.9795) (width 0.7) (layer "B.Cu") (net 18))
 (segment (start 204.4787 95.27) (end 201.0793 98.6694) (width 0.7) (layer "B.Cu") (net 18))
 (segment (start 148.4886 104.3354) (end 147.52 104.3354) (width 0.7) (layer "B.Cu") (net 18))
 (segment (start 159.2129 115.9795) (end 156.6134 113.38) (width 0.7) (layer "B.Cu") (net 18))
 (segment (start 146.7597 110.3724) (end 150.6317 114.2444) (width 0.7) (layer "B.Cu") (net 18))
 (segment (start 156.6134 113.38) (end 156.6134 112.4602) (width 0.7) (layer "B.Cu") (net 18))
 (segment (start 185.5716 115.9795) (end 159.2129 115.9795) (width 0.7) (layer "B.Cu") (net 18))
 (segment (start 150.6317 114.2444) (end 150.6317 117.46) (width 0.7) (layer "B.Cu") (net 18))
 (segment (start 156 113.38) (end 156.6134 113.38) (width 0.7) (layer "B.Cu") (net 18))
 (segment (start 146.7597 105.0957) (end 146.7597 110.3724) (width 0.7) (layer "B.Cu") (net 18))
 (segment (start 148 106) (end 148 107.6317) (width 0.7) (layer "B.Cu") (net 11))
 (segment (start 157.2496 116.8813) (end 148 107.6317) (width 0.7) (layer "B.Cu") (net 11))
 (segment (start 212.5093 99.5643) (end 212.5093 101.196) (width 0.7) (layer "B.Cu") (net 11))
 (segment (start 196.824 116.8813) (end 157.2496 116.8813) (width 0.7) (layer "B.Cu") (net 11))
 (segment (start 212.5093 101.196) (end 196.824 116.8813) (width 0.7) (layer "B.Cu") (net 11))
 (segment (start 160.1883 103.415) (end 147.1266 103.415) (width 0.7) (layer "B.Cu") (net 2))
 (segment (start 145.8333 104.7083) (end 145.8333 119.6956) (width 0.7) (layer "B.Cu") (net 2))
 (segment (start 164 106) (end 162.7733 106) (width 0.7) (layer "B.Cu") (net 2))
 (segment (start 150.1937 124.056) (end 215.0493 124.056) (width 0.7) (layer "B.Cu") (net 2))
 (segment (start 215.0493 122.4243) (end 215.0493 124.056) (width 0.7) (layer "B.Cu") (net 2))
 (segment (start 147.1266 103.415) (end 145.8333 104.7083) (width 0.7) (layer "B.Cu") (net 2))
 (segment (start 162.7733 106) (end 160.1883 103.415) (width 0.7) (layer "B.Cu") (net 2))
 (segment (start 145.8333 119.6956) (end 150.1937 124.056) (width 0.7) (layer "B.Cu") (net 2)))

